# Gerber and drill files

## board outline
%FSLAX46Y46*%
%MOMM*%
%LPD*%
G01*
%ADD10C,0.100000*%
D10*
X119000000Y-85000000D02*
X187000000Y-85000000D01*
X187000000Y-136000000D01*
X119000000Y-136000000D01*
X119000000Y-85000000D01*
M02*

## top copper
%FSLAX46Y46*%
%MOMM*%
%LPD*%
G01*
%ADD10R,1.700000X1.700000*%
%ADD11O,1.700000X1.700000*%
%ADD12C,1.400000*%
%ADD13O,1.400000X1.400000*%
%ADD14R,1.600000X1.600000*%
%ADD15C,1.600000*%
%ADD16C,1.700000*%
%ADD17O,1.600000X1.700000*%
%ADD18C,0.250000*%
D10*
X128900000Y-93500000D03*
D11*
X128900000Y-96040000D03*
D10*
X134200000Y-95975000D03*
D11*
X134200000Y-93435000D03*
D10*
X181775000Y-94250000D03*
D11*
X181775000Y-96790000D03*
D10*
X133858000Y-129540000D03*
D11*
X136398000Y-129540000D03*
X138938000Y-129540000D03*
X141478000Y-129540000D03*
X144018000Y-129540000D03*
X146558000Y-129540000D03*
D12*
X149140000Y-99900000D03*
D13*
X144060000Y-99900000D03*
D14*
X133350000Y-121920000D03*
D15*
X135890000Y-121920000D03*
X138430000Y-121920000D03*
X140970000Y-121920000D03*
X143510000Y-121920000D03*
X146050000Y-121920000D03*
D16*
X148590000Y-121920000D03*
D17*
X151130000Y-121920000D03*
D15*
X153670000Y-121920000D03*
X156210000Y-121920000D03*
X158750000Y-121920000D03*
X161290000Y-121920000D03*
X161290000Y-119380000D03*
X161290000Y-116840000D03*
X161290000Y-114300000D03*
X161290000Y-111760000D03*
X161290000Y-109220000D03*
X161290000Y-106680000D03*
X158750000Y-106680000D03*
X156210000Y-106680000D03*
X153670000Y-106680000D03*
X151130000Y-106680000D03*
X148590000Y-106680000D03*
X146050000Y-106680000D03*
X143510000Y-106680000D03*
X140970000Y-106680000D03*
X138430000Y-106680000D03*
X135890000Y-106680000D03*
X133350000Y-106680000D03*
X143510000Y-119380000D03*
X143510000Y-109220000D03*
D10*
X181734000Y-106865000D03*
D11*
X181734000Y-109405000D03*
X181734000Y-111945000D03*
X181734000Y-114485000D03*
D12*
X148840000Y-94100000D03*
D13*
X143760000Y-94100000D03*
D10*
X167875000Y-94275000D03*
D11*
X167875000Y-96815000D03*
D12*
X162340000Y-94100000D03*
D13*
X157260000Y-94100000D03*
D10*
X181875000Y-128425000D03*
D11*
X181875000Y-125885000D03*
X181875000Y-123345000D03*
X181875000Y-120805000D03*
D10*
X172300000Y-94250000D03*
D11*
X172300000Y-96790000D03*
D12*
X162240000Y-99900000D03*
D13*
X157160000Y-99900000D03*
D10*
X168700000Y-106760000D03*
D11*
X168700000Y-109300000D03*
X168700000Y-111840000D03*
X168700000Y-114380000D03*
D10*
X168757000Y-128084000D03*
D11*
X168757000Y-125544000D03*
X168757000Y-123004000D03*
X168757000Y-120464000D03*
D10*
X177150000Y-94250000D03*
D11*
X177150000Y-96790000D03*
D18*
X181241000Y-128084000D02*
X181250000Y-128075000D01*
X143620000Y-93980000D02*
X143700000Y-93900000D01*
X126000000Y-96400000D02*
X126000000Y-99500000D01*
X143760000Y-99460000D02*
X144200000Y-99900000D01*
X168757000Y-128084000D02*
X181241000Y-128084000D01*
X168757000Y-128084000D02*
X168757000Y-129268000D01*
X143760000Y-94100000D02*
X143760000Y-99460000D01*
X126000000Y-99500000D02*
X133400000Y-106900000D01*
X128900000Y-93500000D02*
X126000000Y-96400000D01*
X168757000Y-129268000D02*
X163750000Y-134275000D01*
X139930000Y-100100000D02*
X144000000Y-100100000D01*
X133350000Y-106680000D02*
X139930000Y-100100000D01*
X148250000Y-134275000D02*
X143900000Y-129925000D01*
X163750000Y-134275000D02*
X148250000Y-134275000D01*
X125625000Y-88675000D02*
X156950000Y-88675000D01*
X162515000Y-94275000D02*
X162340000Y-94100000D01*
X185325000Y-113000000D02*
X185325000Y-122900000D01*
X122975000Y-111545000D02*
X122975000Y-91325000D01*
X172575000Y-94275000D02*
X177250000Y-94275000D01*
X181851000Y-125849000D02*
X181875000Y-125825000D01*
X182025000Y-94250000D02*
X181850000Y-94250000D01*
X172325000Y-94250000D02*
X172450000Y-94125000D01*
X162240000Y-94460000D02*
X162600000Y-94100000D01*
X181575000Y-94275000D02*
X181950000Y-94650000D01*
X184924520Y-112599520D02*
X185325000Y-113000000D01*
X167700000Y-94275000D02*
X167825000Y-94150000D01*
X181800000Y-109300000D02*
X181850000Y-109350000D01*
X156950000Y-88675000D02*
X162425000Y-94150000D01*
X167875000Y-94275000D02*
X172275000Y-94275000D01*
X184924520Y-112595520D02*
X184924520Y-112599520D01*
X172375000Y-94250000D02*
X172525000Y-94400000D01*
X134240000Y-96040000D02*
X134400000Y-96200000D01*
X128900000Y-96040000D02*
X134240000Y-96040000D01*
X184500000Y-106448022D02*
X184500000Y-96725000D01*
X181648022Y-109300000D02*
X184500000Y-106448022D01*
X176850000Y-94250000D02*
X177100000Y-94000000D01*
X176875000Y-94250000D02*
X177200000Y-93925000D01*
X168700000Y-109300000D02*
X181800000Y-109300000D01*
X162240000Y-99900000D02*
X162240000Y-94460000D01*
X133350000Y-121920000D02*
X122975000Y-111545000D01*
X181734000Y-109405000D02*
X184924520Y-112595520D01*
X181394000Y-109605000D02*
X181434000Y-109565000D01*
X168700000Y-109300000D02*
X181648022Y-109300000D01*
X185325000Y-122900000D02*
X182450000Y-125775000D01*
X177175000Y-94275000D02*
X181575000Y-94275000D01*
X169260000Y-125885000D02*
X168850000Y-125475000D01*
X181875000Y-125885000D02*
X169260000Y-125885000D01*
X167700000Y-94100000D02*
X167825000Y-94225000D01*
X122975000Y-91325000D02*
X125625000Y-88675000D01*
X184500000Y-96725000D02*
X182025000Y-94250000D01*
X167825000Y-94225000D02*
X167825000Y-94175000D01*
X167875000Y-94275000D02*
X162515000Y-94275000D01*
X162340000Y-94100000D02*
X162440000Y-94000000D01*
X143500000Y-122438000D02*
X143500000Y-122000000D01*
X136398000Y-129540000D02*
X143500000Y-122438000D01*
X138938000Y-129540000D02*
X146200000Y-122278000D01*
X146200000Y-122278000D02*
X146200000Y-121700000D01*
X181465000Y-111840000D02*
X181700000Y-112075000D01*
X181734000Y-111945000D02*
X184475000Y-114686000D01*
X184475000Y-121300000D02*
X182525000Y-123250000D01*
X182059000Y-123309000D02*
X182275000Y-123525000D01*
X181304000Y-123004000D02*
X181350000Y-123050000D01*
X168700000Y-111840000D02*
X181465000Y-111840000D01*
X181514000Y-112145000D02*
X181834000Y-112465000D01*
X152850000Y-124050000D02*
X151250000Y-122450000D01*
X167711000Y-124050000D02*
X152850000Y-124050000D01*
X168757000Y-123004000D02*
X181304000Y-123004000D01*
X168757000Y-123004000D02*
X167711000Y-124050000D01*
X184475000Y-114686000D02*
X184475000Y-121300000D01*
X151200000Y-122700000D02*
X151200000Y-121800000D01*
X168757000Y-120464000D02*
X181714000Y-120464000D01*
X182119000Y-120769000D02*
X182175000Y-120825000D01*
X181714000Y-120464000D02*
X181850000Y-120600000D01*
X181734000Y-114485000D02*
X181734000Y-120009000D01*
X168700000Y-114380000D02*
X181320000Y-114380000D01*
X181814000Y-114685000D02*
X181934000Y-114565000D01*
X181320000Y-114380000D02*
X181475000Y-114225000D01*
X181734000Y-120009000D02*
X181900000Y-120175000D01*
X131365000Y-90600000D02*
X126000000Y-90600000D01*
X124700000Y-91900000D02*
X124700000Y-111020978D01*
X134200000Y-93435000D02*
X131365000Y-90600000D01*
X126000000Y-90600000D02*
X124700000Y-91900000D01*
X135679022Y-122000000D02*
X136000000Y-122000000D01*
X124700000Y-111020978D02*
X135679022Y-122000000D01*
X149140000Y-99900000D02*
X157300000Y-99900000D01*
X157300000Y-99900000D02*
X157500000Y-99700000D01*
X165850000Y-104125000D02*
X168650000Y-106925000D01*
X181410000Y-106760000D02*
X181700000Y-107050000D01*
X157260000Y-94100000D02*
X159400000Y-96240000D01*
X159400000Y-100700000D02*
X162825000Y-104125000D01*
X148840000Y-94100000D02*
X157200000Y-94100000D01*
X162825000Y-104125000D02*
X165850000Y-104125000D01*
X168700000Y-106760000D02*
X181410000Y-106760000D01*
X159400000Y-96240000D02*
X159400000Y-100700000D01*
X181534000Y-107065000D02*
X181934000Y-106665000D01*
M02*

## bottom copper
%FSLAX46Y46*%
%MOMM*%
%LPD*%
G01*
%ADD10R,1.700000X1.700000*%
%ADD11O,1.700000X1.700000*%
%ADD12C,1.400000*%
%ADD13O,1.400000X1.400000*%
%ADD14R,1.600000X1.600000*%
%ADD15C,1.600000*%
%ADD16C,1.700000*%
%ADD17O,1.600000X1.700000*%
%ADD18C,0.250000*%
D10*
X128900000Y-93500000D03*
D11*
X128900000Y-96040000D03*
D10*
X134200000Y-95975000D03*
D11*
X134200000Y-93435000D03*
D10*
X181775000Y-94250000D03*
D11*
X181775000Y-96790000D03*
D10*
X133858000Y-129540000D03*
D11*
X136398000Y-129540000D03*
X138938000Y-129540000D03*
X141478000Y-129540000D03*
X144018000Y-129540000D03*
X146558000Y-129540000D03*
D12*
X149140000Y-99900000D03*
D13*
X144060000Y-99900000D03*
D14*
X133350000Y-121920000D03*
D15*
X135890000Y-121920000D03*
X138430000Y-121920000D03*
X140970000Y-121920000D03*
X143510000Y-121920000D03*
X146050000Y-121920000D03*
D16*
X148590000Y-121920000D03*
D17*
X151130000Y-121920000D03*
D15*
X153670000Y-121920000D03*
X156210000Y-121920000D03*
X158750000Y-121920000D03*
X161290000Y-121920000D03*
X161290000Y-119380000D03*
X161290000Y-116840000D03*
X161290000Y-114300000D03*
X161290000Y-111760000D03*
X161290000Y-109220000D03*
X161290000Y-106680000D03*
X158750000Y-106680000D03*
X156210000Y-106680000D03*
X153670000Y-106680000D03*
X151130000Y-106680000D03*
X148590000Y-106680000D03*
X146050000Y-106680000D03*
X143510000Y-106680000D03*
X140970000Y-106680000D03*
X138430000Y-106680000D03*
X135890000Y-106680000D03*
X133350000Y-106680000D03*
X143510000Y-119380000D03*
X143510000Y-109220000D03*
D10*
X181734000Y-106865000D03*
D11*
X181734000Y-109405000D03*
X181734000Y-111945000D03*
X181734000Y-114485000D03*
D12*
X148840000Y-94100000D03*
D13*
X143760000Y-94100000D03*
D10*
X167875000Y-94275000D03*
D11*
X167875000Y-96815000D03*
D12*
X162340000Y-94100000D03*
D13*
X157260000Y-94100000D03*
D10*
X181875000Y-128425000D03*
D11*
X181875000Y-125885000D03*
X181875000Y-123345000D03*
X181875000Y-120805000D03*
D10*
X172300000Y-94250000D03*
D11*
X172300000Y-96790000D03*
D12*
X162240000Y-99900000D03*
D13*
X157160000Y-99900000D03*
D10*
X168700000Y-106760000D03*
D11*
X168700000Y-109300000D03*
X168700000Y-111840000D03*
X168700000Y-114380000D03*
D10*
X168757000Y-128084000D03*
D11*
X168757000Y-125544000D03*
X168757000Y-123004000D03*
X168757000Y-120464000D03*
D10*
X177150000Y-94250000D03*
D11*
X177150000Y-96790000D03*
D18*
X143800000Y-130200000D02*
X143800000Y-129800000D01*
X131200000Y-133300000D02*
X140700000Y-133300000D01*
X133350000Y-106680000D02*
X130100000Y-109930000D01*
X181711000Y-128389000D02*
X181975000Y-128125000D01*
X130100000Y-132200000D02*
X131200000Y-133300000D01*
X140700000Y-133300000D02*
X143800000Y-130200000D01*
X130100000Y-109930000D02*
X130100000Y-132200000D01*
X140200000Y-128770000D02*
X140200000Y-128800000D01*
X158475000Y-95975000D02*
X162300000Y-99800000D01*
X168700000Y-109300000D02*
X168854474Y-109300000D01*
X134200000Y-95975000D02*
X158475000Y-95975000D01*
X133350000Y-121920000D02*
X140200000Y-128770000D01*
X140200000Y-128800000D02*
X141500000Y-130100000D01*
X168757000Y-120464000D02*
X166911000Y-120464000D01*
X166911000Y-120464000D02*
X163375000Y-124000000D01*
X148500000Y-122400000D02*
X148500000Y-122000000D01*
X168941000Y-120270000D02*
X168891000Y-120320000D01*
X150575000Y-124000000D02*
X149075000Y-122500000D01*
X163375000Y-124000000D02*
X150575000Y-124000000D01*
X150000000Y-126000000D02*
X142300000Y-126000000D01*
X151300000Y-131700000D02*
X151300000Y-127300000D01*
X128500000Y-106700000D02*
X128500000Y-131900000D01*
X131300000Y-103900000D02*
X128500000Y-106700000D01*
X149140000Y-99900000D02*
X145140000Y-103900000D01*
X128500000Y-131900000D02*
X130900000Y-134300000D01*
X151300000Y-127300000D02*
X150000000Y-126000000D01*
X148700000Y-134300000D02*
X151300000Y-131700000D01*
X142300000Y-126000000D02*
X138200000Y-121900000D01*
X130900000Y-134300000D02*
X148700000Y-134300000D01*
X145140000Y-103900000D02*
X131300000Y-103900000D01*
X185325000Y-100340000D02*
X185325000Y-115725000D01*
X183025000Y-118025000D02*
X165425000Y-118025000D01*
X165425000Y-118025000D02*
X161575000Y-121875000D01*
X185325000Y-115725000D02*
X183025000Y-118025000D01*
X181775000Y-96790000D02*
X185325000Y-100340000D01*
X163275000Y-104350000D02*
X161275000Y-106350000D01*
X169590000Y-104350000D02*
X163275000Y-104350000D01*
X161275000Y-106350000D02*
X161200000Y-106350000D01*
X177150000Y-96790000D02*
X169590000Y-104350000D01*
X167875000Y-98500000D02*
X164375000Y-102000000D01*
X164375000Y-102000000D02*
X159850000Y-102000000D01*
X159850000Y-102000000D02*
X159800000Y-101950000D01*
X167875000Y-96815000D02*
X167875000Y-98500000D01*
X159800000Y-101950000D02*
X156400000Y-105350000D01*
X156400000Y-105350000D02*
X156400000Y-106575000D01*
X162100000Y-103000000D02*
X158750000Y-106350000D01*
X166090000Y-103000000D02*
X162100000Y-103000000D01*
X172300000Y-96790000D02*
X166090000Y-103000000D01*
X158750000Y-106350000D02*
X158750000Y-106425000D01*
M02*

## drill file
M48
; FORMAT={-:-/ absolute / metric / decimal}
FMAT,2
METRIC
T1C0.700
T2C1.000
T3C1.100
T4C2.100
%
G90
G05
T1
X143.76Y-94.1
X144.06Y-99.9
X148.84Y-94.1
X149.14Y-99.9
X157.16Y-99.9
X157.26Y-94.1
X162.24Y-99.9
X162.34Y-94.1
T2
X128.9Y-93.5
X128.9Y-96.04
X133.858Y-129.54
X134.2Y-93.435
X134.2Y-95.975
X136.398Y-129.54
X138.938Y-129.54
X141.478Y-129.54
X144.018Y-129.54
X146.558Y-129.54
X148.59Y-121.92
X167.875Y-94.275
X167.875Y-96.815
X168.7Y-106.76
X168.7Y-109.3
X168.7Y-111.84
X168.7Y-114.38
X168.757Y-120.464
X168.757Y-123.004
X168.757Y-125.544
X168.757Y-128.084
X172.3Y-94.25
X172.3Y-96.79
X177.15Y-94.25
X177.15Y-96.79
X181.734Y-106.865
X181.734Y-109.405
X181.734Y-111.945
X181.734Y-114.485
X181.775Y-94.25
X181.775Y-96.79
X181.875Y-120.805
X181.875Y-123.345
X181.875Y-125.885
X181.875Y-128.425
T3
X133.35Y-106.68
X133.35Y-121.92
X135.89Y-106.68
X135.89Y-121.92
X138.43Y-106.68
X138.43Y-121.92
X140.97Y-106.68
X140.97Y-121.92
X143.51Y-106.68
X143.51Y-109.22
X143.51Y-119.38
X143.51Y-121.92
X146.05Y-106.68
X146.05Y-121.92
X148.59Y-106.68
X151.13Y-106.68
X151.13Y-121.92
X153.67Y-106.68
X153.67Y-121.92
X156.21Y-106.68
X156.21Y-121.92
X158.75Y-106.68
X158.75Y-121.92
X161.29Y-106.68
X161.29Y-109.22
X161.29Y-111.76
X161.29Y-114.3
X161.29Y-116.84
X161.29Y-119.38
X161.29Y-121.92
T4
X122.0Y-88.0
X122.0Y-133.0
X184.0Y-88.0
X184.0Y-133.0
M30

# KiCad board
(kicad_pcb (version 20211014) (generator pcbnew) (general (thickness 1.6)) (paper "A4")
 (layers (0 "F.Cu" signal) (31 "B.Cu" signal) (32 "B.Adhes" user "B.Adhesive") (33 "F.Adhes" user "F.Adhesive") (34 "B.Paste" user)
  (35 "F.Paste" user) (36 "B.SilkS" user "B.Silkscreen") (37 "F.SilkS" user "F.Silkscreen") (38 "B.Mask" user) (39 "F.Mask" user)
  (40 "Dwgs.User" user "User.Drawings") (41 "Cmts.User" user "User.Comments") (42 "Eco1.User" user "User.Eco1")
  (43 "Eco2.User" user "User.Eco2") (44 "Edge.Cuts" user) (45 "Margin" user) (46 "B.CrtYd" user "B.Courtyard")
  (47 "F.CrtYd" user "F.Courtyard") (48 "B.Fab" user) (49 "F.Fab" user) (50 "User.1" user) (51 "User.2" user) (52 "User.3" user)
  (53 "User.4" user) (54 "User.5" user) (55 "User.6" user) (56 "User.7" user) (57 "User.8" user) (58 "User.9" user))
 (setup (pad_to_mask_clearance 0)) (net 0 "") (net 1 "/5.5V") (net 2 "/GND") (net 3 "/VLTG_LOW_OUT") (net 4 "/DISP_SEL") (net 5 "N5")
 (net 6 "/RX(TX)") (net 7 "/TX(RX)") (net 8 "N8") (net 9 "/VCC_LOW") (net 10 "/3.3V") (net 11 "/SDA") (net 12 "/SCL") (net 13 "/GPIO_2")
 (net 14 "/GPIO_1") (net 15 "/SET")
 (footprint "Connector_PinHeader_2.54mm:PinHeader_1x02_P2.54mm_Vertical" (layer "F.Cu") (at 128.9 93.5)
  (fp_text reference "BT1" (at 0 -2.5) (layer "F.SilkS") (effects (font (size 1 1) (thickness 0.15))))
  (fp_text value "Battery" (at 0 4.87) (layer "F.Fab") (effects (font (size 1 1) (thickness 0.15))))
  (pad "1" thru_hole rect locked (at 0 0) (size 1.7 1.7) (drill 1) (layers *.Cu *.Mask) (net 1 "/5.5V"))
  (pad "2" thru_hole oval locked (at 0 2.54) (size 1.7 1.7) (drill 1) (layers *.Cu *.Mask) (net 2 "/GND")))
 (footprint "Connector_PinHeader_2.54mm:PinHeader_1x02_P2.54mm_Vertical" (layer "F.Cu") (at 134.2 95.975 180)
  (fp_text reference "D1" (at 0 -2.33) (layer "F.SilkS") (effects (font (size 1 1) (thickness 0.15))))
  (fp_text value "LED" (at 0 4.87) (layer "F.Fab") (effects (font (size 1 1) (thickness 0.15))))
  (pad "1" thru_hole rect locked (at 0 0 180) (size 1.7 1.7) (drill 1) (layers *.Cu *.Mask) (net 2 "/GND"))
  (pad "2" thru_hole oval locked (at 0 2.54 180) (size 1.7 1.7) (drill 1) (layers *.Cu *.Mask) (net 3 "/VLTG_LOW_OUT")))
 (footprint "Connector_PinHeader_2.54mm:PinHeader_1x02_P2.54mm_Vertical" (layer "F.Cu") (at 181.775 94.25)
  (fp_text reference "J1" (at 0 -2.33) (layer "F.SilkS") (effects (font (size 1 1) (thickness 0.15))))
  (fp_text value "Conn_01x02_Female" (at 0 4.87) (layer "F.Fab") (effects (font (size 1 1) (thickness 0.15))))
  (pad "1" thru_hole rect locked (at 0 0) (size 1.7 1.7) (drill 1) (layers *.Cu *.Mask) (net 2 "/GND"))
  (pad "2" thru_hole oval locked (at 0 2.54) (size 1.7 1.7) (drill 1) (layers *.Cu *.Mask) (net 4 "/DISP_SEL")))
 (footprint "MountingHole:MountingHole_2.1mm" (layer "F.Cu") (at 184 133)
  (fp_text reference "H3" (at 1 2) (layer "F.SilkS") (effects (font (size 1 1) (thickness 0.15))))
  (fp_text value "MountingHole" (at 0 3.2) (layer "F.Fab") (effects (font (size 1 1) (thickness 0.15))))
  (pad "" np_thru_hole circle locked (at 0 0) (size 2.1 2.1) (drill 2.1) (layers *.Cu *.Mask)))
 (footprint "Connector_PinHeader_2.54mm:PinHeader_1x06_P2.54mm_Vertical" (layer "F.Cu") (at 133.858 129.54 90)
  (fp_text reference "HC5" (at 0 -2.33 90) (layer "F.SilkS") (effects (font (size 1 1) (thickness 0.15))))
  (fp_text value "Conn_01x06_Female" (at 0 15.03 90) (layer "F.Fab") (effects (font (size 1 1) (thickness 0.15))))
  (pad "1" thru_hole rect locked (at 0 0 90) (size 1.7 1.7) (drill 1) (layers *.Cu *.Mask) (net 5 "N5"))
  (pad "2" thru_hole oval locked (at 0 2.54 90) (size 1.7 1.7) (drill 1) (layers *.Cu *.Mask) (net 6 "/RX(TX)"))
  (pad "3" thru_hole oval locked (at 0 5.08 90) (size 1.7 1.7) (drill 1) (layers *.Cu *.Mask) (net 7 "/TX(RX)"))
  (pad "4" thru_hole oval locked (at 0 7.62 90) (size 1.7 1.7) (drill 1) (layers *.Cu *.Mask) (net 2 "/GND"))
  (pad "5" thru_hole oval locked (at 0 10.16 90) (size 1.7 1.7) (drill 1) (layers *.Cu *.Mask) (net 1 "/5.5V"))
  (pad "6" thru_hole oval locked (at 0 12.7 90) (size 1.7 1.7) (drill 1) (layers *.Cu *.Mask) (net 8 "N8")))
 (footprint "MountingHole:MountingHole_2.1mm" (layer "F.Cu") (at 122 133)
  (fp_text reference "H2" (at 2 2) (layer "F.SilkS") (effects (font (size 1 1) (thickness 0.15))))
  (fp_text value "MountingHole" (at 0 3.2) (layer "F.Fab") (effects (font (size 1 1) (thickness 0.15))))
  (pad "" np_thru_hole circle locked (at 0 0) (size 2.1 2.1) (drill 2.1) (layers *.Cu *.Mask)))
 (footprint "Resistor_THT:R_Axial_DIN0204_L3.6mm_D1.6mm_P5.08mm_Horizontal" (layer "F.Cu") (at 149.14 99.9 180)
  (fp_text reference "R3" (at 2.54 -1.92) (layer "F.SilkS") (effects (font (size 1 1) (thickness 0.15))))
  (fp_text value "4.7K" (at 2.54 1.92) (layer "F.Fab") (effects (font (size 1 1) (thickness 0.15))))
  (pad "1" thru_hole circle locked (at 0 0 180) (size 1.4 1.4) (drill 0.7) (layers *.Cu *.Mask) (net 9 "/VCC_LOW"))
  (pad "2" thru_hole oval locked (at 5.08 0 180) (size 1.4 1.4) (drill 0.7) (layers *.Cu *.Mask) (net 1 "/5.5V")))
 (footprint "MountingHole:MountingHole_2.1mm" (layer "F.Cu") (at 184 88)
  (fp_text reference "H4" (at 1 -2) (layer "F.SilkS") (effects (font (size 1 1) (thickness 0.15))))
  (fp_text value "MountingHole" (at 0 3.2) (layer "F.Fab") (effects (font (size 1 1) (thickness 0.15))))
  (pad "" np_thru_hole circle locked (at 0 0) (size 2.1 2.1) (drill 2.1) (layers *.Cu *.Mask)))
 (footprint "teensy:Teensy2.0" (layer "F.Cu") (at 147.32 114.3)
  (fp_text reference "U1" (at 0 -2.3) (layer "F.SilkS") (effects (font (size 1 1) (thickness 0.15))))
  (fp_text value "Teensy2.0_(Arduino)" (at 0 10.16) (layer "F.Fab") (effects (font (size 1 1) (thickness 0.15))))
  (pad "1" thru_hole rect locked (at -13.97 7.62) (size 1.6 1.6) (drill 1.1) (layers *.Cu *.Mask))
  (pad "2" thru_hole circle locked (at -11.43 7.62) (size 1.6 1.6) (drill 1.1) (layers *.Cu *.Mask))
  (pad "3" thru_hole circle locked (at -8.89 7.62) (size 1.6 1.6) (drill 1.1) (layers *.Cu *.Mask))
  (pad "4" thru_hole circle locked (at -6.35 7.62) (size 1.6 1.6) (drill 1.1) (layers *.Cu *.Mask))
  (pad "5" thru_hole circle locked (at -3.81 7.62) (size 1.6 1.6) (drill 1.1) (layers *.Cu *.Mask))
  (pad "6" thru_hole circle locked (at -1.27 7.62) (size 1.6 1.6) (drill 1.1) (layers *.Cu *.Mask))
  (pad "7" thru_hole circle locked (at 1.27 7.62) (size 1.7 1.7) (drill 1) (layers *.Cu *.Mask))
  (pad "8" thru_hole oval locked (at 3.81 7.62) (size 1.6 1.7) (drill 1.1) (layers *.Cu *.Mask))
  (pad "9" thru_hole circle locked (at 6.35 7.62) (size 1.6 1.6) (drill 1.1) (layers *.Cu *.Mask))
  (pad "10" thru_hole circle locked (at 8.89 7.62) (size 1.6 1.6) (drill 1.1) (layers *.Cu *.Mask))
  (pad "11" thru_hole circle locked (at 11.43 7.62) (size 1.6 1.6) (drill 1.1) (layers *.Cu *.Mask))
  (pad "12" thru_hole circle locked (at 13.97 7.62) (size 1.6 1.6) (drill 1.1) (layers *.Cu *.Mask))
  (pad "13" thru_hole circle locked (at 13.97 5.08) (size 1.6 1.6) (drill 1.1) (layers *.Cu *.Mask))
  (pad "14" thru_hole circle locked (at 13.97 2.54) (size 1.6 1.6) (drill 1.1) (layers *.Cu *.Mask))
  (pad "15" thru_hole circle locked (at 13.97 0) (size 1.6 1.6) (drill 1.1) (layers *.Cu *.Mask))
  (pad "16" thru_hole circle locked (at 13.97 -2.54) (size 1.6 1.6) (drill 1.1) (layers *.Cu *.Mask))
  (pad "17" thru_hole circle locked (at 13.97 -5.08) (size 1.6 1.6) (drill 1.1) (layers *.Cu *.Mask))
  (pad "18" thru_hole circle locked (at 13.97 -7.62) (size 1.6 1.6) (drill 1.1) (layers *.Cu *.Mask))
  (pad "19" thru_hole circle locked (at 11.43 -7.62) (size 1.6 1.6) (drill 1.1) (layers *.Cu *.Mask))
  (pad "20" thru_hole circle locked (at 8.89 -7.62) (size 1.6 1.6) (drill 1.1) (layers *.Cu *.Mask))
  (pad "21" thru_hole circle locked (at 6.35 -7.62) (size 1.6 1.6) (drill 1.1) (layers *.Cu *.Mask))
  (pad "22" thru_hole circle locked (at 3.81 -7.62) (size 1.6 1.6) (drill 1.1) (layers *.Cu *.Mask))
  (pad "23" thru_hole circle locked (at 1.27 -7.62) (size 1.6 1.6) (drill 1.1) (layers *.Cu *.Mask))
  (pad "24" thru_hole circle locked (at -1.27 -7.62) (size 1.6 1.6) (drill 1.1) (layers *.Cu *.Mask))
  (pad "25" thru_hole circle locked (at -3.81 -7.62) (size 1.6 1.6) (drill 1.1) (layers *.Cu *.Mask))
  (pad "26" thru_hole circle locked (at -6.35 -7.62) (size 1.6 1.6) (drill 1.1) (layers *.Cu *.Mask))
  (pad "27" thru_hole circle locked (at -8.89 -7.62) (size 1.6 1.6) (drill 1.1) (layers *.Cu *.Mask))
  (pad "28" thru_hole circle locked (at -11.43 -7.62) (size 1.6 1.6) (drill 1.1) (layers *.Cu *.Mask))
  (pad "29" thru_hole circle locked (at -13.97 -7.62) (size 1.6 1.6) (drill 1.1) (layers *.Cu *.Mask))
  (pad "30" thru_hole circle locked (at -3.81 5.08) (size 1.6 1.6) (drill 1.1) (layers *.Cu *.Mask))
  (pad "31" thru_hole circle locked (at -3.81 -5.08) (size 1.6 1.6) (drill 1.1) (layers *.Cu *.Mask)))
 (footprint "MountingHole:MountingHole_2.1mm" (layer "F.Cu") (at 122 88)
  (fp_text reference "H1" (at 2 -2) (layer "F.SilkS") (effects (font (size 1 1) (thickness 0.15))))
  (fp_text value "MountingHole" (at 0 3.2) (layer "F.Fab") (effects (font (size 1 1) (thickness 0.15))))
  (pad "" np_thru_hole circle locked (at 0 0) (size 2.1 2.1) (drill 2.1) (layers *.Cu *.Mask)))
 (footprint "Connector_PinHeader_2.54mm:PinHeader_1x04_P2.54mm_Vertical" (layer "F.Cu") (at 181.734 106.865)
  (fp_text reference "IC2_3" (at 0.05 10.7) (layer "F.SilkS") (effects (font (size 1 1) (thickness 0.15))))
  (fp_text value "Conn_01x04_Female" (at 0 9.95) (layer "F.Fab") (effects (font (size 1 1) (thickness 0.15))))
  (pad "1" thru_hole rect locked (at 0 0) (size 1.7 1.7) (drill 1) (layers *.Cu *.Mask) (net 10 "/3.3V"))
  (pad "2" thru_hole oval locked (at 0 2.54) (size 1.7 1.7) (drill 1) (layers *.Cu *.Mask) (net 2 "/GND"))
  (pad "3" thru_hole oval locked (at 0 5.08) (size 1.7 1.7) (drill 1) (layers *.Cu *.Mask) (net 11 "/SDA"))
  (pad "4" thru_hole oval locked (at 0 7.62) (size 1.7 1.7) (drill 1) (layers *.Cu *.Mask) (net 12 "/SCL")))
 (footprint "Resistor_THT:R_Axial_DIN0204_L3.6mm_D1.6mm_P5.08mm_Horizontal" (layer "F.Cu") (at 148.84 94.1 180)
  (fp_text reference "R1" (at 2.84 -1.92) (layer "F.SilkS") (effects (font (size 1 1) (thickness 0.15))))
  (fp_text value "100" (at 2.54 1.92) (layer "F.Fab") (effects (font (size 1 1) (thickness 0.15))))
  (pad "1" thru_hole circle locked (at 0 0 180) (size 1.4 1.4) (drill 0.7) (layers *.Cu *.Mask))
  (pad "2" thru_hole oval locked (at 5.08 0 180) (size 1.4 1.4) (drill 0.7) (layers *.Cu *.Mask)))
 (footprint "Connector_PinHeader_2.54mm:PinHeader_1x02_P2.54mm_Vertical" (layer "F.Cu") (at 167.875 94.275)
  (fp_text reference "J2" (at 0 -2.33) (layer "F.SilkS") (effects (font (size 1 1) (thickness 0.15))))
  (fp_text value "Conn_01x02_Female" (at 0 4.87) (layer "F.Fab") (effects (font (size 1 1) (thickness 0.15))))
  (pad "1" thru_hole rect locked (at 0 0) (size 1.7 1.7) (drill 1) (layers *.Cu *.Mask) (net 2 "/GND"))
  (pad "2" thru_hole oval locked (at 0 2.54) (size 1.7 1.7) (drill 1) (layers *.Cu *.Mask) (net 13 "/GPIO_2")))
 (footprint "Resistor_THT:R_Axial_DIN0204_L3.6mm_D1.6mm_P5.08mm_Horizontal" (layer "F.Cu") (at 162.34 94.1 180)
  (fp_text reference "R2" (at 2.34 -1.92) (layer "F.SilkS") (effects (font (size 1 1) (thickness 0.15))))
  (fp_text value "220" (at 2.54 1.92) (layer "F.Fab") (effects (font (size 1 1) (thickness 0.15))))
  (pad "1" thru_hole circle locked (at 0 0 180) (size 1.4 1.4) (drill 0.7) (layers *.Cu *.Mask) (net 2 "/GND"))
  (pad "2" thru_hole oval locked (at 5.08 0 180) (size 1.4 1.4) (drill 0.7) (layers *.Cu *.Mask) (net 10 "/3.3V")))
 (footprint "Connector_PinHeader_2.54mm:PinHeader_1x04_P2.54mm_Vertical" (layer "F.Cu") (at 181.875 128.425 180)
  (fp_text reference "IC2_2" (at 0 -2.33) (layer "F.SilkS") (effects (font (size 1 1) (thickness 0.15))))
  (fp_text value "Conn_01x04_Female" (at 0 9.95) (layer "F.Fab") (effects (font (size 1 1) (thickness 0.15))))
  (pad "1" thru_hole rect locked (at 0 0 180) (size 1.7 1.7) (drill 1) (layers *.Cu *.Mask) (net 1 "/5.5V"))
  (pad "2" thru_hole oval locked (at 0 2.54 180) (size 1.7 1.7) (drill 1) (layers *.Cu *.Mask) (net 2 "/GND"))
  (pad "3" thru_hole oval locked (at 0 5.08 180) (size 1.7 1.7) (drill 1) (layers *.Cu *.Mask) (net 11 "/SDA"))
  (pad "4" thru_hole oval locked (at 0 7.62 180) (size 1.7 1.7) (drill 1) (layers *.Cu *.Mask) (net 12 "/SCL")))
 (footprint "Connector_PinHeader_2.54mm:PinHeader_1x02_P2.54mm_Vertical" (layer "F.Cu") (at 172.3 94.25)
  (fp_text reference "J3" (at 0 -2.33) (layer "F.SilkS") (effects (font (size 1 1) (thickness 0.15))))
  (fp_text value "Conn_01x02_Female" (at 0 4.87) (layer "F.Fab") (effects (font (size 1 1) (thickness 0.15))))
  (pad "1" thru_hole rect locked (at 0 0) (size 1.7 1.7) (drill 1) (layers *.Cu *.Mask) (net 2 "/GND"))
  (pad "2" thru_hole oval locked (at 0 2.54) (size 1.7 1.7) (drill 1) (layers *.Cu *.Mask) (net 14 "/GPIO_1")))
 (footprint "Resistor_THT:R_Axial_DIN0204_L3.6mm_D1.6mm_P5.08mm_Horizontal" (layer "F.Cu") (at 162.24 99.9 180)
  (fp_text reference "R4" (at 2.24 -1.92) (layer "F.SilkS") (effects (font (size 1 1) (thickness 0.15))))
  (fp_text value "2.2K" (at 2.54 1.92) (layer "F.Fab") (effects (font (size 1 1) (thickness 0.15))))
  (pad "1" thru_hole circle locked (at 0 0 180) (size 1.4 1.4) (drill 0.7) (layers *.Cu *.Mask) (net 2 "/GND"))
  (pad "2" thru_hole oval locked (at 5.08 0 180) (size 1.4 1.4) (drill 0.7) (layers *.Cu *.Mask) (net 9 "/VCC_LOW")))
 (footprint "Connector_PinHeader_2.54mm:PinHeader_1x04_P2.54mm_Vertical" (layer "F.Cu") (at 168.7 106.76)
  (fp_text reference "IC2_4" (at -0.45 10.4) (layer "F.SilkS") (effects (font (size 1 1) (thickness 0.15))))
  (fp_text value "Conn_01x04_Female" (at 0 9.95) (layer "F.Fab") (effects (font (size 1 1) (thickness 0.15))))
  (pad "1" thru_hole rect locked (at 0 0) (size 1.7 1.7) (drill 1) (layers *.Cu *.Mask) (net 10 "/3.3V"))
  (pad "2" thru_hole oval locked (at 0 2.54) (size 1.7 1.7) (drill 1) (layers *.Cu *.Mask) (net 2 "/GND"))
  (pad "3" thru_hole oval locked (at 0 5.08) (size 1.7 1.7) (drill 1) (layers *.Cu *.Mask) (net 11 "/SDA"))
  (pad "4" thru_hole oval locked (at 0 7.62) (size 1.7 1.7) (drill 1) (layers *.Cu *.Mask) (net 12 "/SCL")))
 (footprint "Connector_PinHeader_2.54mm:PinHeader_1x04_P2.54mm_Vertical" (layer "F.Cu") (at 168.757 128.084 180)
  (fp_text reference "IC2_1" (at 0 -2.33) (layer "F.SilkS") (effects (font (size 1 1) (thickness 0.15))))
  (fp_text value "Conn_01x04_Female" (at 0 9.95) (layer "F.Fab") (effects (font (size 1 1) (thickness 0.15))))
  (pad "1" thru_hole rect locked (at 0 0 180) (size 1.7 1.7) (drill 1) (layers *.Cu *.Mask) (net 1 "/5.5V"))
  (pad "2" thru_hole oval locked (at 0 2.54 180) (size 1.7 1.7) (drill 1) (layers *.Cu *.Mask) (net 2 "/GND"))
  (pad "3" thru_hole oval locked (at 0 5.08 180) (size 1.7 1.7) (drill 1) (layers *.Cu *.Mask) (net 11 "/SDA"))
  (pad "4" thru_hole oval locked (at 0 7.62 180) (size 1.7 1.7) (drill 1) (layers *.Cu *.Mask) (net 12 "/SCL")))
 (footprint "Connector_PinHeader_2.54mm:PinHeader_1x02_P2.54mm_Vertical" (layer "F.Cu") (at 177.15 94.25)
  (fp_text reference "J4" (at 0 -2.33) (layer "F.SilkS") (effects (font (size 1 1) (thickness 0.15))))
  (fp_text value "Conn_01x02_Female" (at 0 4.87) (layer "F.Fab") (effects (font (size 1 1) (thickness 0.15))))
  (pad "1" thru_hole rect locked (at 0 0) (size 1.7 1.7) (drill 1) (layers *.Cu *.Mask) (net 2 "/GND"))
  (pad "2" thru_hole oval locked (at 0 2.54) (size 1.7 1.7) (drill 1) (layers *.Cu *.Mask) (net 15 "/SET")))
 (gr_rect (start 119 85) (end 187 136) (layer "Edge.Cuts") (width 0.1) (fill none))
 (segment (start 181.241 128.084) (end 181.25 128.075) (width 0.25) (layer "F.Cu") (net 1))
 (segment (start 143.62 93.98) (end 143.7 93.9) (width 0.25) (layer "F.Cu") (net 1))
 (segment (start 126 96.4) (end 126 99.5) (width 0.25) (layer "F.Cu") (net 1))
 (segment (start 143.76 99.46) (end 144.2 99.9) (width 0.25) (layer "F.Cu") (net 1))
 (segment (start 168.757 128.084) (end 181.241 128.084) (width 0.25) (layer "F.Cu") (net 1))
 (segment (start 168.757 128.084) (end 168.757 129.268) (width 0.25) (layer "F.Cu") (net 1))
 (segment (start 143.76 94.1) (end 143.76 99.46) (width 0.25) (layer "F.Cu") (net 1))
 (segment (start 126 99.5) (end 133.4 106.9) (width 0.25) (layer "F.Cu") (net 1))
 (segment (start 128.9 93.5) (end 126 96.4) (width 0.25) (layer "F.Cu") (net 1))
 (segment (start 168.757 129.268) (end 163.75 134.275) (width 0.25) (layer "F.Cu") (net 1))
 (segment (start 139.93 100.1) (end 144 100.1) (width 0.25) (layer "F.Cu") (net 1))
 (segment (start 133.35 106.68) (end 139.93 100.1) (width 0.25) (layer "F.Cu") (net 1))
 (segment (start 148.25 134.275) (end 143.9 129.925) (width 0.25) (layer "F.Cu") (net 1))
 (segment (start 163.75 134.275) (end 148.25 134.275) (width 0.25) (layer "F.Cu") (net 1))
 (segment (start 143.8 130.2) (end 143.8 129.8) (width 0.25) (layer "B.Cu") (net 1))
 (segment (start 131.2 133.3) (end 140.7 133.3) (width 0.25) (layer "B.Cu") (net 1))
 (segment (start 133.35 106.68) (end 130.1 109.93) (width 0.25) (layer "B.Cu") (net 1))
 (segment (start 181.711 128.389) (end 181.975 128.125) (width 0.25) (layer "B.Cu") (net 1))
 (segment (start 130.1 132.2) (end 131.2 133.3) (width 0.25) (layer "B.Cu") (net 1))
 (segment (start 140.7 133.3) (end 143.8 130.2) (width 0.25) (layer "B.Cu") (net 1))
 (segment (start 130.1 109.93) (end 130.1 132.2) (width 0.25) (layer "B.Cu") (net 1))
 (segment (start 125.625 88.675) (end 156.95 88.675) (width 0.25) (layer "F.Cu") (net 2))
 (segment (start 162.515 94.275) (end 162.34 94.1) (width 0.25) (layer "F.Cu") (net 2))
 (segment (start 185.325 113) (end 185.325 122.9) (width 0.25) (layer "F.Cu") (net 2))
 (segment (start 122.975 111.545) (end 122.975 91.325) (width 0.25) (layer "F.Cu") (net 2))
 (segment (start 172.575 94.275) (end 177.25 94.275) (width 0.25) (layer "F.Cu") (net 2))
 (segment (start 181.851 125.849) (end 181.875 125.825) (width 0.25) (layer "F.Cu") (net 2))
 (segment (start 182.025 94.25) (end 181.85 94.25) (width 0.25) (layer "F.Cu") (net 2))
 (segment (start 172.325 94.25) (end 172.45 94.125) (width 0.25) (layer "F.Cu") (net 2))
 (segment (start 162.24 94.46) (end 162.6 94.1) (width 0.25) (layer "F.Cu") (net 2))
 (segment (start 181.575 94.275) (end 181.95 94.65) (width 0.25) (layer "F.Cu") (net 2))
 (segment (start 184.92452 112.59952) (end 185.325 113) (width 0.25) (layer "F.Cu") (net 2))
 (segment (start 167.7 94.275) (end 167.825 94.15) (width 0.25) (layer "F.Cu") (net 2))
 (segment (start 181.8 109.3) (end 181.85 109.35) (width 0.25) (layer "F.Cu") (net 2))
 (segment (start 156.95 88.675) (end 162.425 94.15) (width 0.25) (layer "F.Cu") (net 2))
 (segment (start 167.875 94.275) (end 172.275 94.275) (width 0.25) (layer "F.Cu") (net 2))
 (segment (start 184.92452 112.59552) (end 184.92452 112.59952) (width 0.25) (layer "F.Cu") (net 2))
 (segment (start 172.375 94.25) (end 172.525 94.4) (width 0.25) (layer "F.Cu") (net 2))
 (segment (start 134.24 96.04) (end 134.4 96.2) (width 0.25) (layer "F.Cu") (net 2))
 (segment (start 128.9 96.04) (end 134.24 96.04) (width 0.25) (layer "F.Cu") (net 2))
 (segment (start 184.5 106.448022) (end 184.5 96.725) (width 0.25) (layer "F.Cu") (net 2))
 (segment (start 181.648022 109.3) (end 184.5 106.448022) (width 0.25) (layer "F.Cu") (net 2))
 (segment (start 176.85 94.25) (end 177.1 94) (width 0.25) (layer "F.Cu") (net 2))
 (segment (start 176.875 94.25) (end 177.2 93.925) (width 0.25) (layer "F.Cu") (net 2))
 (segment (start 168.7 109.3) (end 181.8 109.3) (width 0.25) (layer "F.Cu") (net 2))
 (segment (start 162.24 99.9) (end 162.24 94.46) (width 0.25) (layer "F.Cu") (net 2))
 (segment (start 133.35 121.92) (end 122.975 111.545) (width 0.25) (layer "F.Cu") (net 2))
 (segment (start 181.734 109.405) (end 184.92452 112.59552) (width 0.25) (layer "F.Cu") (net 2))
 (segment (start 181.394 109.605) (end 181.434 109.565) (width 0.25) (layer "F.Cu") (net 2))
 (segment (start 168.7 109.3) (end 181.648022 109.3) (width 0.25) (layer "F.Cu") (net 2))
 (segment (start 185.325 122.9) (end 182.45 125.775) (width 0.25) (layer "F.Cu") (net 2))
 (segment (start 177.175 94.275) (end 181.575 94.275) (width 0.25) (layer "F.Cu") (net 2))
 (segment (start 169.26 125.885) (end 168.85 125.475) (width 0.25) (layer "F.Cu") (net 2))
 (segment (start 181.875 125.885) (end 169.26 125.885) (width 0.25) (layer "F.Cu") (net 2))
 (segment (start 167.7 94.1) (end 167.825 94.225) (width 0.25) (layer "F.Cu") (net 2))
 (segment (start 122.975 91.325) (end 125.625 88.675) (width 0.25) (layer "F.Cu") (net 2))
 (segment (start 184.5 96.725) (end 182.025 94.25) (width 0.25) (layer "F.Cu") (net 2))
 (segment (start 167.825 94.225) (end 167.825 94.175) (width 0.25) (layer "F.Cu") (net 2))
 (segment (start 167.875 94.275) (end 162.515 94.275) (width 0.25) (layer "F.Cu") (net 2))
 (segment (start 162.34 94.1) (end 162.44 94) (width 0.25) (layer "F.Cu") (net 2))
 (segment (start 140.2 128.77) (end 140.2 128.8) (width 0.25) (layer "B.Cu") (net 2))
 (segment (start 158.475 95.975) (end 162.3 99.8) (width 0.25) (layer "B.Cu") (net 2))
 (segment (start 168.7 109.3) (end 168.854474 109.3) (width 0.25) (layer "B.Cu") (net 2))
 (segment (start 134.2 95.975) (end 158.475 95.975) (width 0.25) (layer "B.Cu") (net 2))
 (segment (start 133.35 121.92) (end 140.2 128.77) (width 0.25) (layer "B.Cu") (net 2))
 (segment (start 140.2 128.8) (end 141.5 130.1) (width 0.25) (layer "B.Cu") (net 2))
 (segment (start 143.5 122.438) (end 143.5 122) (width 0.25) (layer "F.Cu") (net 6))
 (segment (start 136.398 129.54) (end 143.5 122.438) (width 0.25) (layer "F.Cu") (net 6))
 (segment (start 138.938 129.54) (end 146.2 122.278) (width 0.25) (layer "F.Cu") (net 7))
 (segment (start 146.2 122.278) (end 146.2 121.7) (width 0.25) (layer "F.Cu") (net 7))
 (segment (start 181.465 111.84) (end 181.7 112.075) (width 0.25) (layer "F.Cu") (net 11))
 (segment (start 181.734 111.945) (end 184.475 114.686) (width 0.25) (layer "F.Cu") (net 11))
 (segment (start 184.475 121.3) (end 182.525 123.25) (width 0.25) (layer "F.Cu") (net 11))
 (segment (start 182.059 123.309) (end 182.275 123.525) (width 0.25) (layer "F.Cu") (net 11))
 (segment (start 181.304 123.004) (end 181.35 123.05) (width 0.25) (layer "F.Cu") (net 11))
 (segment (start 168.7 111.84) (end 181.465 111.84) (width 0.25) (layer "F.Cu") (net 11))
 (segment (start 181.514 112.145) (end 181.834 112.465) (width 0.25) (layer "F.Cu") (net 11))
 (segment (start 152.85 124.05) (end 151.25 122.45) (width 0.25) (layer "F.Cu") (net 11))
 (segment (start 167.711 124.05) (end 152.85 124.05) (width 0.25) (layer "F.Cu") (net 11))
 (segment (start 168.757 123.004) (end 181.304 123.004) (width 0.25) (layer "F.Cu") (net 11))
 (segment (start 168.757 123.004) (end 167.711 124.05) (width 0.25) (layer "F.Cu") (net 11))
 (segment (start 184.475 114.686) (end 184.475 121.3) (width 0.25) (layer "F.Cu") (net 11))
 (segment (start 151.2 122.7) (end 151.2 121.8) (width 0.25) (layer "F.Cu") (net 11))
 (segment (start 168.757 120.464) (end 181.714 120.464) (width 0.25) (layer "F.Cu") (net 12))
 (segment (start 182.119 120.769) (end 182.175 120.825) (width 0.25) (layer "F.Cu") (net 12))
 (segment (start 181.714 120.464) (end 181.85 120.6) (width 0.25) (layer "F.Cu") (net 12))
 (segment (start 181.734 114.485) (end 181.734 120.009) (width 0.25) (layer "F.Cu") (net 12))
 (segment (start 168.7 114.38) (end 181.32 114.38) (width 0.25) (layer "F.Cu") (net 12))
 (segment (start 181.814 114.685) (end 181.934 114.565) (width 0.25) (layer "F.Cu") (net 12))
 (segment (start 181.32 114.38) (end 181.475 114.225) (width 0.25) (layer "F.Cu") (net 12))
 (segment (start 181.734 120.009) (end 181.9 120.175) (width 0.25) (layer "F.Cu") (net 12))
 (segment (start 168.757 120.464) (end 166.911 120.464) (width 0.25) (layer "B.Cu") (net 12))
 (segment (start 166.911 120.464) (end 163.375 124) (width 0.25) (layer "B.Cu") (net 12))
 (segment (start 148.5 122.4) (end 148.5 122) (width 0.25) (layer "B.Cu") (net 12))
 (segment (start 168.941 120.27) (end 168.891 120.32) (width 0.25) (layer "B.Cu") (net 12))
 (segment (start 150.575 124) (end 149.075 122.5) (width 0.25) (layer "B.Cu") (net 12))
 (segment (start 163.375 124) (end 150.575 124) (width 0.25) (layer "B.Cu") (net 12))
 (segment (start 131.365 90.6) (end 126 90.6) (width 0.25) (layer "F.Cu") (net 3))
 (segment (start 124.7 91.9) (end 124.7 111.020978) (width 0.25) (layer "F.Cu") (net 3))
 (segment (start 134.2 93.435) (end 131.365 90.6) (width 0.25) (layer "F.Cu") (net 3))
 (segment (start 126 90.6) (end 124.7 91.9) (width 0.25) (layer "F.Cu") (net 3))
 (segment (start 135.679022 122) (end 136 122) (width 0.25) (layer "F.Cu") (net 3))
 (segment (start 124.7 111.020978) (end 135.679022 122) (width 0.25) (layer "F.Cu") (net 3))
 (segment (start 149.14 99.9) (end 157.3 99.9) (width 0.25) (layer "F.Cu") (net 9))
 (segment (start 157.3 99.9) (end 157.5 99.7) (width 0.25) (layer "F.Cu") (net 9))
 (segment (start 150 126) (end 142.3 126) (width 0.25) (layer "B.Cu") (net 9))
 (segment (start 151.3 131.7) (end 151.3 127.3) (width 0.25) (layer "B.Cu") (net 9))
 (segment (start 128.5 106.7) (end 128.5 131.9) (width 0.25) (layer "B.Cu") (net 9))
 (segment (start 131.3 103.9) (end 128.5 106.7) (width 0.25) (layer "B.Cu") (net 9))
 (segment (start 149.14 99.9) (end 145.14 103.9) (width 0.25) (layer "B.Cu") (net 9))
 (segment (start 128.5 131.9) (end 130.9 134.3) (width 0.25) (layer "B.Cu") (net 9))
 (segment (start 151.3 127.3) (end 150 126) (width 0.25) (layer "B.Cu") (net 9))
 (segment (start 148.7 134.3) (end 151.3 131.7) (width 0.25) (layer "B.Cu") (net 9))
 (segment (start 142.3 126) (end 138.2 121.9) (width 0.25) (layer "B.Cu") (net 9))
 (segment (start 130.9 134.3) (end 148.7 134.3) (width 0.25) (layer "B.Cu") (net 9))
 (segment (start 145.14 103.9) (end 131.3 103.9) (width 0.25) (layer "B.Cu") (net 9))
 (segment (start 185.325 100.34) (end 185.325 115.725) (width 0.25) (layer "B.Cu") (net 4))
 (segment (start 183.025 118.025) (end 165.425 118.025) (width 0.25) (layer "B.Cu") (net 4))
 (segment (start 165.425 118.025) (end 161.575 121.875) (width 0.25) (layer "B.Cu") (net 4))
 (segment (start 185.325 115.725) (end 183.025 118.025) (width 0.25) (layer "B.Cu") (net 4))
 (segment (start 181.775 96.79) (end 185.325 100.34) (width 0.25) (layer "B.Cu") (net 4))
 (segment (start 163.275 104.35) (end 161.275 106.35) (width 0.25) (layer "B.Cu") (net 15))
 (segment (start 169.59 104.35) (end 163.275 104.35) (width 0.25) (layer "B.Cu") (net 15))
 (segment (start 161.275 106.35) (end 161.2 106.35) (width 0.25) (layer "B.Cu") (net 15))
 (segment (start 177.15 96.79) (end 169.59 104.35) (width 0.25) (layer "B.Cu") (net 15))
 (segment (start 167.875 98.5) (end 164.375 102) (width 0.25) (layer "B.Cu") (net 13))
 (segment (start 164.375 102) (end 159.85 102) (width 0.25) (layer "B.Cu") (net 13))
 (segment (start 159.85 102) (end 159.8 101.95) (width 0.25) (layer "B.Cu") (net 13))
 (segment (start 167.875 96.815) (end 167.875 98.5) (width 0.25) (layer "B.Cu") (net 13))
 (segment (start 159.8 101.95) (end 156.4 105.35) (width 0.25) (layer "B.Cu") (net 13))
 (segment (start 156.4 105.35) (end 156.4 106.575) (width 0.25) (layer "B.Cu") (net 13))
 (segment (start 162.1 103) (end 158.75 106.35) (width 0.25) (layer "B.Cu") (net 14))
 (segment (start 166.09 103) (end 162.1 103) (width 0.25) (layer "B.Cu") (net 14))
 (segment (start 172.3 96.79) (end 166.09 103) (width 0.25) (layer "B.Cu") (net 14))
 (segment (start 158.75 106.35) (end 158.75 106.425) (width 0.25) (layer "B.Cu") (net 14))
 (segment (start 165.85 104.125) (end 168.65 106.925) (width 0.25) (layer "F.Cu") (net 10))
 (segment (start 181.41 106.76) (end 181.7 107.05) (width 0.25) (layer "F.Cu") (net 10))
 (segment (start 157.26 94.1) (end 159.4 96.24) (width 0.25) (layer "F.Cu") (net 10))
 (segment (start 159.4 100.7) (end 162.825 104.125) (width 0.25) (layer "F.Cu") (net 10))
 (segment (start 148.84 94.1) (end 157.2 94.1) (width 0.25) (layer "F.Cu") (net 10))
 (segment (start 162.825 104.125) (end 165.85 104.125) (width 0.25) (layer "F.Cu") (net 10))
 (segment (start 168.7 106.76) (end 181.41 106.76) (width 0.25) (layer "F.Cu") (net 10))
 (segment (start 159.4 96.24) (end 159.4 100.7) (width 0.25) (layer "F.Cu") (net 10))
 (segment (start 181.534 107.065) (end 181.934 106.665) (width 0.25) (layer "F.Cu") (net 10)))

